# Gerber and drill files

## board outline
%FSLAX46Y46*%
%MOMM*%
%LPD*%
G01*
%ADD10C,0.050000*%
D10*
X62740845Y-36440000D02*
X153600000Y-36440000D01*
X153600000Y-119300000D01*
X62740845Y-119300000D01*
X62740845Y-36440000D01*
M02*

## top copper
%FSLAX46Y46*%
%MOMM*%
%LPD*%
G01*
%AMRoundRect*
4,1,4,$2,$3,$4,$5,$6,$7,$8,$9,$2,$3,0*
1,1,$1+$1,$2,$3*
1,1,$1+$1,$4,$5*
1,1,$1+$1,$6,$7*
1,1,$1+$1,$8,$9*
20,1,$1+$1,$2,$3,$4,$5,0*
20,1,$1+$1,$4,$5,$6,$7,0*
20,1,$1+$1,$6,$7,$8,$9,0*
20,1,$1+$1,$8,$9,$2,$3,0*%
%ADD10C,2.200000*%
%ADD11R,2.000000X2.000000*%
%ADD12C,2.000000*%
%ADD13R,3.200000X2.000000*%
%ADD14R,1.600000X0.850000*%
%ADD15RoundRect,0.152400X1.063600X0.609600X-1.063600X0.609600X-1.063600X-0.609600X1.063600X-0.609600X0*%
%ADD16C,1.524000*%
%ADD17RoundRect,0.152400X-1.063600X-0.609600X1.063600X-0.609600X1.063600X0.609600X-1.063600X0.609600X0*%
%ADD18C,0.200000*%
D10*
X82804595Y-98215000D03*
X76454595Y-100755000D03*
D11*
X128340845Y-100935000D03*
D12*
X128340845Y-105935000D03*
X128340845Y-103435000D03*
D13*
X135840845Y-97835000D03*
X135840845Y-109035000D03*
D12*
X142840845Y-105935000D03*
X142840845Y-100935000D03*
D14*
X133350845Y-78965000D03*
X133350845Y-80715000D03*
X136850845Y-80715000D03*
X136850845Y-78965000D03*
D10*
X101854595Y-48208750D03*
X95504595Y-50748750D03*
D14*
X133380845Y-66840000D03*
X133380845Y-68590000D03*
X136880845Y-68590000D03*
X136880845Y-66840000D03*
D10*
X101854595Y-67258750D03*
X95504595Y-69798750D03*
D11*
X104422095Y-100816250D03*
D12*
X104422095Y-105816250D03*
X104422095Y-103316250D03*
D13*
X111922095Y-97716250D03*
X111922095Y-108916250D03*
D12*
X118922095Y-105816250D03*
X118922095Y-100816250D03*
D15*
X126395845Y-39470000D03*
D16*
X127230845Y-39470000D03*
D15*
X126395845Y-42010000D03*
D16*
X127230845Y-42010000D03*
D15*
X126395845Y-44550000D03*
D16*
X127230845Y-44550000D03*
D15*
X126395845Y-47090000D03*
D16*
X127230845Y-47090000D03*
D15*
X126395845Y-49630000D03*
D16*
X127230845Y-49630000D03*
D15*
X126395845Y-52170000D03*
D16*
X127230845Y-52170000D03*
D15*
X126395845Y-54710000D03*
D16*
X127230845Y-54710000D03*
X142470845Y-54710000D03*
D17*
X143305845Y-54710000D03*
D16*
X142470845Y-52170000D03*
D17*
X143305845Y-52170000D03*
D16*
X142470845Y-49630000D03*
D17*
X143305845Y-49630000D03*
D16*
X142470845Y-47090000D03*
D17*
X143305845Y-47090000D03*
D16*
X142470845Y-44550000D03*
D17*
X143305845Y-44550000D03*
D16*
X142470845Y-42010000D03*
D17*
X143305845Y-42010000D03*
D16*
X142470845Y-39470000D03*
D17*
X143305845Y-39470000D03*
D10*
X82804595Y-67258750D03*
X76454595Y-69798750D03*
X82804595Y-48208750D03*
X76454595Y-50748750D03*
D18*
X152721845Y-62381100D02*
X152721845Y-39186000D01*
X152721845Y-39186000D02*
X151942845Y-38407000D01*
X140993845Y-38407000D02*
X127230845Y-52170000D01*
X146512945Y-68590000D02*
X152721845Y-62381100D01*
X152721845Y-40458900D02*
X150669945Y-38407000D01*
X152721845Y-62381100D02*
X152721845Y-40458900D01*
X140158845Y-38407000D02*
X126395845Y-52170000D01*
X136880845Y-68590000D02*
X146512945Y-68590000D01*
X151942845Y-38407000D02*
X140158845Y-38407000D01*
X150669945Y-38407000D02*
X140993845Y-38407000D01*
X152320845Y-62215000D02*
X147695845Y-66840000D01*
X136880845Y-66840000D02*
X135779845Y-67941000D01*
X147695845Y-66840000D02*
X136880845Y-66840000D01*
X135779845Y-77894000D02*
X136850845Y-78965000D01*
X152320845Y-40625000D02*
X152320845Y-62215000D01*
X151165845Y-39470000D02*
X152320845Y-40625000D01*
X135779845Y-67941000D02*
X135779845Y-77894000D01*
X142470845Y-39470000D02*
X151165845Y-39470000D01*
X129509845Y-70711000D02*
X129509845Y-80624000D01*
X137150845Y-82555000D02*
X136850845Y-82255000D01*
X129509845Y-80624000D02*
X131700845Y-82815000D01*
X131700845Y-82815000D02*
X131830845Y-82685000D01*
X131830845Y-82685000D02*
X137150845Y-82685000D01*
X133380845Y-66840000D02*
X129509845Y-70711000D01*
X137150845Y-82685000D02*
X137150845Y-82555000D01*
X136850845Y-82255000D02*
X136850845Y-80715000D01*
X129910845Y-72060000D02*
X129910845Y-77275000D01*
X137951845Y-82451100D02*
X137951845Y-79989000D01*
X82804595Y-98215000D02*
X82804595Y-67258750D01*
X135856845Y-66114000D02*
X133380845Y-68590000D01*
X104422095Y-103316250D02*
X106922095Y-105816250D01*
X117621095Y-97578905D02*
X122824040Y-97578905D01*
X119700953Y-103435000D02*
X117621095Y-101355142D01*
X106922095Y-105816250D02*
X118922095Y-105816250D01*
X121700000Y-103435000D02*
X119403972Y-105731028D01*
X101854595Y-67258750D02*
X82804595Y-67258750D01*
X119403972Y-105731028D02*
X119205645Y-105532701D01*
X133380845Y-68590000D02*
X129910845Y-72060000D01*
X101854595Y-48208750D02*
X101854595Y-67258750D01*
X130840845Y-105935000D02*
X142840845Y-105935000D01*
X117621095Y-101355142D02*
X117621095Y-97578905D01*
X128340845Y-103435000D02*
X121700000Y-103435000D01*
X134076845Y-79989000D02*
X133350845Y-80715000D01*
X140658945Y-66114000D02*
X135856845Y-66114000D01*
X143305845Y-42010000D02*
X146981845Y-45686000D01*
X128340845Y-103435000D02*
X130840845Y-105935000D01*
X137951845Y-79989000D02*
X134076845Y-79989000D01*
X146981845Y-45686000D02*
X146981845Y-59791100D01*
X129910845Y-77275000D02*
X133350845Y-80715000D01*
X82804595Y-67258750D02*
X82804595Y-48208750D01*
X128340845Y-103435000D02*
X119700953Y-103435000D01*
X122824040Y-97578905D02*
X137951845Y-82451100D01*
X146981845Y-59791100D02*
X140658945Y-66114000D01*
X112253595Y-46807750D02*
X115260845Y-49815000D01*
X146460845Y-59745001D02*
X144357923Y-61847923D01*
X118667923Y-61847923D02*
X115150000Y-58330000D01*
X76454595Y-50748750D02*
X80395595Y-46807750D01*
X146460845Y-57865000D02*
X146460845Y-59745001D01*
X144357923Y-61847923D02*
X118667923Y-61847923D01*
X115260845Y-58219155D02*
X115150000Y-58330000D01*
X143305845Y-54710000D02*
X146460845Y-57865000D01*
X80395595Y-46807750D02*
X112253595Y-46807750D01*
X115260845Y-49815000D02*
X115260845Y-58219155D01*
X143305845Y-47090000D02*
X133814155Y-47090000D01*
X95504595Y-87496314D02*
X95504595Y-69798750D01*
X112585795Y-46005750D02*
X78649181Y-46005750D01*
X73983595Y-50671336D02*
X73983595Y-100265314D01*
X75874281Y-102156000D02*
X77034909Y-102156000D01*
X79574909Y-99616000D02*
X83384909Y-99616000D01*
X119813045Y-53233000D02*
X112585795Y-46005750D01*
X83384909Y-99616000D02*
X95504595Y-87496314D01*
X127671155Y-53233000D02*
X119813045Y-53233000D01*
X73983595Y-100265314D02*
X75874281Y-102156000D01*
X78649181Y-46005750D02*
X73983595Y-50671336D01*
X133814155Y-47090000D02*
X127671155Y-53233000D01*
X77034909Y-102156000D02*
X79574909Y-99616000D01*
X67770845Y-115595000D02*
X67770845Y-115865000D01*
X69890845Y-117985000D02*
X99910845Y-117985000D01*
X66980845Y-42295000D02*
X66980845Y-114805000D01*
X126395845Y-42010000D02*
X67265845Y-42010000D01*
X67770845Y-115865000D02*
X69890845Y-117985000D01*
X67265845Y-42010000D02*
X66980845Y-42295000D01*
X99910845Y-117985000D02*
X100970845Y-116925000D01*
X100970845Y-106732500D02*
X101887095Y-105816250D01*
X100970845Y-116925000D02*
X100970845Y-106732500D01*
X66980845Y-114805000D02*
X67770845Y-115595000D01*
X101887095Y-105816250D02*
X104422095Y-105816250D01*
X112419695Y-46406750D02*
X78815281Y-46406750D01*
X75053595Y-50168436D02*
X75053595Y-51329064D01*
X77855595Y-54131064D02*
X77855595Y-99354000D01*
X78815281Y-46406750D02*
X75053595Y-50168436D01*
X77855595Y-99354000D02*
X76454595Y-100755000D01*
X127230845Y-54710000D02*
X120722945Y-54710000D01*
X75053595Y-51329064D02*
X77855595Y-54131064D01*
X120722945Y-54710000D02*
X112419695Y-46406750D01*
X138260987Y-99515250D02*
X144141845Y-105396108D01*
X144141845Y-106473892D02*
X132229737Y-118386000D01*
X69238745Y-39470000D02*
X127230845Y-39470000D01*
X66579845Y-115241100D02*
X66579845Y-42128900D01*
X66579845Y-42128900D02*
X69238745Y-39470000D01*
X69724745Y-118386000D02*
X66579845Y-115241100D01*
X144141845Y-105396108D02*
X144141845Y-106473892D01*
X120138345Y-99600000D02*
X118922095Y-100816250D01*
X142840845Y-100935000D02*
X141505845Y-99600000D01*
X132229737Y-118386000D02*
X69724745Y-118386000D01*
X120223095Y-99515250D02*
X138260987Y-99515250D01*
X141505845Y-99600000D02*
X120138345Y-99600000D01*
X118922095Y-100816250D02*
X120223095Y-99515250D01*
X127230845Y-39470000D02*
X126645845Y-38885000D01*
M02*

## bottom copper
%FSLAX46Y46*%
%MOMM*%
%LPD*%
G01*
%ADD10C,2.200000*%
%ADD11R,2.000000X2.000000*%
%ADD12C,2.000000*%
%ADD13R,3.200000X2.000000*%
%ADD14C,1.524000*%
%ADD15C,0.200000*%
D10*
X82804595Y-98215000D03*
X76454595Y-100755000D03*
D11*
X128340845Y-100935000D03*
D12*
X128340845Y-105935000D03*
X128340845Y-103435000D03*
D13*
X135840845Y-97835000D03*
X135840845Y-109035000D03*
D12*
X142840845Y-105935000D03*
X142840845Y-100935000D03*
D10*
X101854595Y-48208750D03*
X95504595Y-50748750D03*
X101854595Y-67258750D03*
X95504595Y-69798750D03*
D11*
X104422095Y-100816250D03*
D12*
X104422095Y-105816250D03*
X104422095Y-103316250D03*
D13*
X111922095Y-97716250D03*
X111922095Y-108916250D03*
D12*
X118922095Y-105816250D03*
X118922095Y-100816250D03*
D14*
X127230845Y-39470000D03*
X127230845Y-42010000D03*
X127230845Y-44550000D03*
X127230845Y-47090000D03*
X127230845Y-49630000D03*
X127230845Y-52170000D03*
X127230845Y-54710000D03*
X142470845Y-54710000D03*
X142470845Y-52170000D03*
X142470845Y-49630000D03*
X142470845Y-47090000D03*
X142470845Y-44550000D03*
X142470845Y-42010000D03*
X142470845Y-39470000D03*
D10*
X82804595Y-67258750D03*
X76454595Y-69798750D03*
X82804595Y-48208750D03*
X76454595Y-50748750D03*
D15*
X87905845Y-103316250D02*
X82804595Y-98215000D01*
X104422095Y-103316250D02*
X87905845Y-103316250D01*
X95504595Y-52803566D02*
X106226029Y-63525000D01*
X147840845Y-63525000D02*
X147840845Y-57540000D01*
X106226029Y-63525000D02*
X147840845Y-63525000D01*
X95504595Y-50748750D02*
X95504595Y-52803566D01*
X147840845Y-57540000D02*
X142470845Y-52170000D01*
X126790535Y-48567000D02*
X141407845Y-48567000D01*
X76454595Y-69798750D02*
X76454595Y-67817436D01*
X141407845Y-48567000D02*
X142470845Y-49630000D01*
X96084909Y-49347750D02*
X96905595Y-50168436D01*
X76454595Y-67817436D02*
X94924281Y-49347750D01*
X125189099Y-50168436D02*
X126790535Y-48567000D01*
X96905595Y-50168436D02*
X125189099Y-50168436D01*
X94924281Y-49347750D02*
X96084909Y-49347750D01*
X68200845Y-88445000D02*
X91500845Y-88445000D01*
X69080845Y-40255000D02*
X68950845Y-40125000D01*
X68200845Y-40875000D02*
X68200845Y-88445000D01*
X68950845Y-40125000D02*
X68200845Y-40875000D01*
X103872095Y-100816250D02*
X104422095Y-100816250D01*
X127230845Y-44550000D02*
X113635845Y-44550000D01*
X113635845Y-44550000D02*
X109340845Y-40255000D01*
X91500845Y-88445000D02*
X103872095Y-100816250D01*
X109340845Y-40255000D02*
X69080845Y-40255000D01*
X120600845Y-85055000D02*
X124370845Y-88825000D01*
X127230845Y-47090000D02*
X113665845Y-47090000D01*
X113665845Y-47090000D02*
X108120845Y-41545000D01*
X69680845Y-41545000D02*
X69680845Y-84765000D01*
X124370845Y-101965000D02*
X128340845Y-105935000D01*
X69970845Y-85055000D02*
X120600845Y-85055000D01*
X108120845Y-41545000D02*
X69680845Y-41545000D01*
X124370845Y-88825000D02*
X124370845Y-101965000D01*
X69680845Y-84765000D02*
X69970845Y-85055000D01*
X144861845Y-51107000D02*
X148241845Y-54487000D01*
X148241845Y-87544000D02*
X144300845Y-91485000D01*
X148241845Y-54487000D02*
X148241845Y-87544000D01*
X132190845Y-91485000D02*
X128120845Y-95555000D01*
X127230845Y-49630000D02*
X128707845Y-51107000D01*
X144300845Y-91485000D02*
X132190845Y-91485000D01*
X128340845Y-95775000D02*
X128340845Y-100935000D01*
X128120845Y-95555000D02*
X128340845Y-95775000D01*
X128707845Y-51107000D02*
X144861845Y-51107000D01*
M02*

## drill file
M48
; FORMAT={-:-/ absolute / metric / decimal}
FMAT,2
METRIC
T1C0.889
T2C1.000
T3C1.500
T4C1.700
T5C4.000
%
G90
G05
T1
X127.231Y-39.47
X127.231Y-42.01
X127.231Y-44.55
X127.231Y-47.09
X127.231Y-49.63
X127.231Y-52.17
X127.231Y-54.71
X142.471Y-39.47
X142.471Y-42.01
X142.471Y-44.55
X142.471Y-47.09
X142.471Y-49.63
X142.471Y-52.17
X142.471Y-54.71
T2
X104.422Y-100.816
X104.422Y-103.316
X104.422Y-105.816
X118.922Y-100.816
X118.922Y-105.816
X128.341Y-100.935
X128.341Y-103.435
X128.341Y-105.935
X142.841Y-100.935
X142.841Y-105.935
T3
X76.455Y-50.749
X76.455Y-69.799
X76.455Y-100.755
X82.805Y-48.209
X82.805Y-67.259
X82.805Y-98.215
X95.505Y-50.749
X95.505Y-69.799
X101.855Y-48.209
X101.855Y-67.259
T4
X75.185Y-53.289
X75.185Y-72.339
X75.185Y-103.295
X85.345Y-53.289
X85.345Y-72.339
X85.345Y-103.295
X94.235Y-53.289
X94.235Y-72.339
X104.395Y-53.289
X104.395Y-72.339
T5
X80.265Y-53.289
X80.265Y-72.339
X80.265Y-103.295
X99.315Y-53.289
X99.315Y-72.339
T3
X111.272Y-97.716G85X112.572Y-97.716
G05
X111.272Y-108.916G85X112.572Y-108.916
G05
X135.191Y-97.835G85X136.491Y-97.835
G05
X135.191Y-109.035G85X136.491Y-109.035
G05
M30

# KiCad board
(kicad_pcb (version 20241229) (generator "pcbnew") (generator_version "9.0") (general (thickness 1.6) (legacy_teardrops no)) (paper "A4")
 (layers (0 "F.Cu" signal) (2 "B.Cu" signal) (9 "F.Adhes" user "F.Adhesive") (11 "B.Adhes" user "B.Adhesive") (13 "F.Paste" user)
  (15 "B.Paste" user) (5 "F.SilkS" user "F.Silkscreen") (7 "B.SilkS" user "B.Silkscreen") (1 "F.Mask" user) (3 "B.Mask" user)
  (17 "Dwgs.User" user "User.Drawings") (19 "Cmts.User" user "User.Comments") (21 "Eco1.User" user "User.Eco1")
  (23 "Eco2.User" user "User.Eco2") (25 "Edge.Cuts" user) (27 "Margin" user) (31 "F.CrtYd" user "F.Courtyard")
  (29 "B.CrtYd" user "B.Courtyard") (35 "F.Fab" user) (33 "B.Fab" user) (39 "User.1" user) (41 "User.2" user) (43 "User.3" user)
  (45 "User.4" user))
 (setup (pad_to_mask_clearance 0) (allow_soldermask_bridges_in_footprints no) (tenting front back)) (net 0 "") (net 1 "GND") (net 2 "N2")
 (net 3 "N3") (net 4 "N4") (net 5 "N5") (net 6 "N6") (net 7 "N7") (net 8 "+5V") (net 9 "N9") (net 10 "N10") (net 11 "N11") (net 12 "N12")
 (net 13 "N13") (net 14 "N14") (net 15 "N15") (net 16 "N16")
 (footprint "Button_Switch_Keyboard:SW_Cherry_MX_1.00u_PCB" (layer "F.Cu") (at 82.804595 98.215)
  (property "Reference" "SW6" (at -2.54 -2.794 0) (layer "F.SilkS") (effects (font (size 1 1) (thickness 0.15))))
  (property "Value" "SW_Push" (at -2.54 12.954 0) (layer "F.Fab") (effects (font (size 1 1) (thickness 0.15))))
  (pad "" np_thru_hole circle (at -7.62 5.08) (size 1.7 1.7) (drill 1.7) (layers "*.Cu" "*.Mask"))
  (pad "" np_thru_hole circle (at -2.54 5.08) (size 4 4) (drill 4) (layers "*.Cu" "*.Mask"))
  (pad "" np_thru_hole circle (at 2.54 5.08) (size 1.7 1.7) (drill 1.7) (layers "*.Cu" "*.Mask"))
  (pad "1" thru_hole circle (at 0 0) (size 2.2 2.2) (drill 1.5) (layers "*.Cu" "*.Mask") (remove_unused_layers no) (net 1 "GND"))
  (pad "2" thru_hole circle (at -6.35 2.54) (size 2.2 2.2) (drill 1.5) (layers "*.Cu" "*.Mask") (remove_unused_layers no) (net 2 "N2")))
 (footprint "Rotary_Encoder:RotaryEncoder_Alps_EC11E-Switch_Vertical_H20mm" (layer "F.Cu") (at 128.340845 100.935)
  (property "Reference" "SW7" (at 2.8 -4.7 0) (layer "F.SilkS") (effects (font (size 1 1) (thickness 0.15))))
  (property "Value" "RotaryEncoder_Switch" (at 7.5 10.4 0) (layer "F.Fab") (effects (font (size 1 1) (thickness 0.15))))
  (pad "A" thru_hole rect (at 0 0) (size 2 2) (drill 1) (layers "*.Cu" "*.Mask") (remove_unused_layers no) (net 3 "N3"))
  (pad "B" thru_hole circle (at 0 5) (size 2 2) (drill 1) (layers "*.Cu" "*.Mask") (remove_unused_layers no) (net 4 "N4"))
  (pad "C" thru_hole circle (at 0 2.5) (size 2 2) (drill 1) (layers "*.Cu" "*.Mask") (remove_unused_layers no) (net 1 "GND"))
  (pad "MP" thru_hole rect (at 7.5 -3.1) (size 3.2 2) (drill oval 2.8 1.5) (layers "*.Cu" "*.Mask") (remove_unused_layers no))
  (pad "MP" thru_hole rect (at 7.5 8.1) (size 3.2 2) (drill oval 2.8 1.5) (layers "*.Cu" "*.Mask") (remove_unused_layers no))
  (pad "S1" thru_hole circle (at 14.5 5) (size 2 2) (drill 1) (layers "*.Cu" "*.Mask") (remove_unused_layers no) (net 1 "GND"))
  (pad "S2" thru_hole circle (at 14.5 0) (size 2 2) (drill 1) (layers "*.Cu" "*.Mask") (remove_unused_layers no) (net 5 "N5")))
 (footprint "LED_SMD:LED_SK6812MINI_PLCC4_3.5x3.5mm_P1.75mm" (layer "F.Cu") (at 135.100845 79.84)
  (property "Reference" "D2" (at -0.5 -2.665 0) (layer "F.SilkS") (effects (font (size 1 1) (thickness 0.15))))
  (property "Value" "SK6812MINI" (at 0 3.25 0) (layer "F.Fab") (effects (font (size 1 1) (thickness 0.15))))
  (pad "1" smd rect (at -1.75 -0.875) (size 1.6 0.85) (layers "F.Cu" "F.Mask" "F.Paste") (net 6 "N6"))
  (pad "2" smd rect (at -1.75 0.875) (size 1.6 0.85) (layers "F.Cu" "F.Mask" "F.Paste") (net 1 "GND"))
  (pad "3" smd rect (at 1.75 0.875) (size 1.6 0.85) (layers "F.Cu" "F.Mask" "F.Paste") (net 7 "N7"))
  (pad "4" smd rect (at 1.75 -0.875) (size 1.6 0.85) (layers "F.Cu" "F.Mask" "F.Paste") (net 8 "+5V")))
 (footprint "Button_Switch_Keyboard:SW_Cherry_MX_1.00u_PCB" (layer "F.Cu") (at 101.854595 48.20875)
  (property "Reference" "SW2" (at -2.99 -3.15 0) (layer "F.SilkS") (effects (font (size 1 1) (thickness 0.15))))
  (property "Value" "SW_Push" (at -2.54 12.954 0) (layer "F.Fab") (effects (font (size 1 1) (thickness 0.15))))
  (pad "" np_thru_hole circle (at -7.62 5.08) (size 1.7 1.7) (drill 1.7) (layers "*.Cu" "*.Mask"))
  (pad "" np_thru_hole circle (at -2.54 5.08) (size 4 4) (drill 4) (layers "*.Cu" "*.Mask"))
  (pad "" np_thru_hole circle (at 2.54 5.08) (size 1.7 1.7) (drill 1.7) (layers "*.Cu" "*.Mask"))
  (pad "1" thru_hole circle (at 0 0) (size 2.2 2.2) (drill 1.5) (layers "*.Cu" "*.Mask") (remove_unused_layers no) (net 1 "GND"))
  (pad "2" thru_hole circle (at -6.35 2.54) (size 2.2 2.2) (drill 1.5) (layers "*.Cu" "*.Mask") (remove_unused_layers no) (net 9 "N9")))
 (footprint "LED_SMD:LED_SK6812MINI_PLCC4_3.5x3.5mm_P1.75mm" (layer "F.Cu") (at 135.130845 67.715)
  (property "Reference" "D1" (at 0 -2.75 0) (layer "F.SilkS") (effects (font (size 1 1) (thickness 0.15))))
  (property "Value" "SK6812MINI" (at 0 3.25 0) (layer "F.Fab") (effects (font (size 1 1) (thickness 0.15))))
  (pad "1" smd rect (at -1.75 -0.875) (size 1.6 0.85) (layers "F.Cu" "F.Mask" "F.Paste") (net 7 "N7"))
  (pad "2" smd rect (at -1.75 0.875) (size 1.6 0.85) (layers "F.Cu" "F.Mask" "F.Paste") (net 1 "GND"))
  (pad "3" smd rect (at 1.75 0.875) (size 1.6 0.85) (layers "F.Cu" "F.Mask" "F.Paste") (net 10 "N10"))
  (pad "4" smd rect (at 1.75 -0.875) (size 1.6 0.85) (layers "F.Cu" "F.Mask" "F.Paste") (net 8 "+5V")))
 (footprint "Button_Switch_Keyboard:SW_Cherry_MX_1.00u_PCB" (layer "F.Cu") (at 101.854595 67.25875)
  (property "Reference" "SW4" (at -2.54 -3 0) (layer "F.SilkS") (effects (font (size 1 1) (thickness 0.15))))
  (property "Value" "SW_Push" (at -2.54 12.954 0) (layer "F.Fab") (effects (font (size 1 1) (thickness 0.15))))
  (pad "" np_thru_hole circle (at -7.62 5.08) (size 1.7 1.7) (drill 1.7) (layers "*.Cu" "*.Mask"))
  (pad "" np_thru_hole circle (at -2.54 5.08) (size 4 4) (drill 4) (layers "*.Cu" "*.Mask"))
  (pad "" np_thru_hole circle (at 2.54 5.08) (size 1.7 1.7) (drill 1.7) (layers "*.Cu" "*.Mask"))
  (pad "1" thru_hole circle (at 0 0) (size 2.2 2.2) (drill 1.5) (layers "*.Cu" "*.Mask") (remove_unused_layers no) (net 1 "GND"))
  (pad "2" thru_hole circle (at -6.35 2.54) (size 2.2 2.2) (drill 1.5) (layers "*.Cu" "*.Mask") (remove_unused_layers no) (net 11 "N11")))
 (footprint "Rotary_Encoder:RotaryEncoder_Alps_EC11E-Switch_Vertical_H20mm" (layer "F.Cu") (at 104.422095 100.81625)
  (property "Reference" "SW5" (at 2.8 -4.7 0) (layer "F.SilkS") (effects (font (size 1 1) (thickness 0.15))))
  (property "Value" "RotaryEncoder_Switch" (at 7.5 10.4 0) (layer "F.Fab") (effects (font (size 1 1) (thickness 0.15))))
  (pad "A" thru_hole rect (at 0 0) (size 2 2) (drill 1) (layers "*.Cu" "*.Mask") (remove_unused_layers no) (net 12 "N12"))
  (pad "B" thru_hole circle (at 0 5) (size 2 2) (drill 1) (layers "*.Cu" "*.Mask") (remove_unused_layers no) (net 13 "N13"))
  (pad "C" thru_hole circle (at 0 2.5) (size 2 2) (drill 1) (layers "*.Cu" "*.Mask") (remove_unused_layers no) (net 1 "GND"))
  (pad "MP" thru_hole rect (at 7.5 -3.1) (size 3.2 2) (drill oval 2.8 1.5) (layers "*.Cu" "*.Mask") (remove_unused_layers no))
  (pad "MP" thru_hole rect (at 7.5 8.1) (size 3.2 2) (drill oval 2.8 1.5) (layers "*.Cu" "*.Mask") (remove_unused_layers no))
  (pad "S1" thru_hole circle (at 14.5 5) (size 2 2) (drill 1) (layers "*.Cu" "*.Mask") (remove_unused_layers no) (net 1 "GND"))
  (pad "S2" thru_hole circle (at 14.5 0) (size 2 2) (drill 1) (layers "*.Cu" "*.Mask") (remove_unused_layers no) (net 5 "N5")))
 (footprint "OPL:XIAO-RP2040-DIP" (layer "F.Cu") (at 134.850845 47.09)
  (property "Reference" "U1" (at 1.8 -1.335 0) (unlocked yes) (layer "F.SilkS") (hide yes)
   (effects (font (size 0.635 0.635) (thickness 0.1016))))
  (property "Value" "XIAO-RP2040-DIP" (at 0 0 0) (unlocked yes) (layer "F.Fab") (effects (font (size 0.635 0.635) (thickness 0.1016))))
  (pad "1" smd roundrect (at -8.455 -7.62 180) (size 2.432 1.524) (layers "F.Cu" "F.Mask") (roundrect_rratio 0.1) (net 5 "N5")
   (thermal_bridge_angle 45))
  (pad "1" thru_hole circle (at -7.62 -7.62 180) (size 1.524 1.524) (drill 0.889) (layers "*.Cu" "*.Mask") (remove_unused_layers no)
   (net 5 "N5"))
  (pad "2" smd roundrect (at -8.455 -5.08 180) (size 2.432 1.524) (layers "F.Cu" "F.Mask") (roundrect_rratio 0.1) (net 13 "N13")
   (thermal_bridge_angle 45))
  (pad "2" thru_hole circle (at -7.62 -5.08 180) (size 1.524 1.524) (drill 0.889) (layers "*.Cu" "*.Mask") (remove_unused_layers no)
   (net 13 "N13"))
  (pad "3" smd roundrect (at -8.455 -2.54 180) (size 2.432 1.524) (layers "F.Cu" "F.Mask") (roundrect_rratio 0.1) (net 12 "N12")
   (thermal_bridge_angle 45))
  (pad "3" thru_hole circle (at -7.62 -2.54 180) (size 1.524 1.524) (drill 0.889) (layers "*.Cu" "*.Mask") (remove_unused_layers no)
   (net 12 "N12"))
  (pad "4" smd roundrect (at -8.455 0 180) (size 2.432 1.524) (layers "F.Cu" "F.Mask") (roundrect_rratio 0.1) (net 4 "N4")
   (thermal_bridge_angle 45))
  (pad "4" thru_hole circle (at -7.62 0 180) (size 1.524 1.524) (drill 0.889) (layers "*.Cu" "*.Mask") (remove_unused_layers no)
   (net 4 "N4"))
  (pad "5" smd roundrect (at -8.455 2.54 180) (size 2.432 1.524) (layers "F.Cu" "F.Mask") (roundrect_rratio 0.1) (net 3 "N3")
   (thermal_bridge_angle 45))
  (pad "5" thru_hole circle (at -7.62 2.54 180) (size 1.524 1.524) (drill 0.889) (layers "*.Cu" "*.Mask") (remove_unused_layers no)
   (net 3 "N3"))
  (pad "6" smd roundrect (at -8.455 5.08 180) (size 2.432 1.524) (layers "F.Cu" "F.Mask") (roundrect_rratio 0.1) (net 10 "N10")
   (thermal_bridge_angle 45))
  (pad "6" thru_hole circle (at -7.62 5.08 180) (size 1.524 1.524) (drill 0.889) (layers "*.Cu" "*.Mask") (remove_unused_layers no)
   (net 10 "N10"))
  (pad "7" smd roundrect (at -8.455 7.62 180) (size 2.432 1.524) (layers "F.Cu" "F.Mask") (roundrect_rratio 0.1) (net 2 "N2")
   (thermal_bridge_angle 45))
  (pad "7" thru_hole circle (at -7.62 7.62 180) (size 1.524 1.524) (drill 0.889) (layers "*.Cu" "*.Mask") (remove_unused_layers no)
   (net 2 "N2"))
  (pad "8" thru_hole circle (at 7.62 7.62) (size 1.524 1.524) (drill 0.889) (layers "*.Cu" "*.Mask") (remove_unused_layers no)
   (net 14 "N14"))
  (pad "8" smd roundrect (at 8.455 7.62) (size 2.432 1.524) (layers "F.Cu" "F.Mask") (roundrect_rratio 0.1) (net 14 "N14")
   (thermal_bridge_angle 45))
  (pad "9" thru_hole circle (at 7.62 5.08) (size 1.524 1.524) (drill 0.889) (layers "*.Cu" "*.Mask") (remove_unused_layers no) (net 9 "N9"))
  (pad "9" smd roundrect (at 8.455 5.08) (size 2.432 1.524) (layers "F.Cu" "F.Mask") (roundrect_rratio 0.1) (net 9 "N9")
   (thermal_bridge_angle 45))
  (pad "10" thru_hole circle (at 7.62 2.54) (size 1.524 1.524) (drill 0.889) (layers "*.Cu" "*.Mask") (remove_unused_layers no)
   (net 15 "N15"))
  (pad "10" smd roundrect (at 8.455 2.54) (size 2.432 1.524) (layers "F.Cu" "F.Mask") (roundrect_rratio 0.1) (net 15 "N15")
   (thermal_bridge_angle 45))
  (pad "11" thru_hole circle (at 7.62 0) (size 1.524 1.524) (drill 0.889) (layers "*.Cu" "*.Mask") (remove_unused_layers no) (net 11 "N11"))
  (pad "11" smd roundrect (at 8.455 0) (size 2.432 1.524) (layers "F.Cu" "F.Mask") (roundrect_rratio 0.1) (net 11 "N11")
   (thermal_bridge_angle 45))
  (pad "12" thru_hole circle (at 7.62 -2.54) (size 1.524 1.524) (drill 0.889) (layers "*.Cu" "*.Mask") (remove_unused_layers no)
   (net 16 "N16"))
  (pad "12" smd roundrect (at 8.455 -2.54) (size 2.432 1.524) (layers "F.Cu" "F.Mask") (roundrect_rratio 0.1) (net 16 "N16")
   (thermal_bridge_angle 45))
  (pad "13" thru_hole circle (at 7.62 -5.08) (size 1.524 1.524) (drill 0.889) (layers "*.Cu" "*.Mask") (remove_unused_layers no)
   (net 1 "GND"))
  (pad "13" smd roundrect (at 8.455 -5.08) (size 2.432 1.524) (layers "F.Cu" "F.Mask") (roundrect_rratio 0.1) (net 1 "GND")
   (thermal_bridge_angle 45))
  (pad "14" thru_hole circle (at 7.62 -7.62) (size 1.524 1.524) (drill 0.889) (layers "*.Cu" "*.Mask") (remove_unused_layers no)
   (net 8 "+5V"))
  (pad "14" smd roundrect (at 8.455 -7.62) (size 2.432 1.524) (layers "F.Cu" "F.Mask") (roundrect_rratio 0.1) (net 8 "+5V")
   (thermal_bridge_angle 45)))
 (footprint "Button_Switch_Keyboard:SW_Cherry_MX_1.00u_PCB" (layer "F.Cu") (at 82.804595 67.25875)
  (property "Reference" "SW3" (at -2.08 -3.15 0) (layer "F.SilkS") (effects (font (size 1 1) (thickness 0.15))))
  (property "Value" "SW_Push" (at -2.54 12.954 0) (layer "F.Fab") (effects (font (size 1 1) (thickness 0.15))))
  (pad "" np_thru_hole circle (at -7.62 5.08) (size 1.7 1.7) (drill 1.7) (layers "*.Cu" "*.Mask"))
  (pad "" np_thru_hole circle (at -2.54 5.08) (size 4 4) (drill 4) (layers "*.Cu" "*.Mask"))
  (pad "" np_thru_hole circle (at 2.54 5.08) (size 1.7 1.7) (drill 1.7) (layers "*.Cu" "*.Mask"))
  (pad "1" thru_hole circle (at 0 0) (size 2.2 2.2) (drill 1.5) (layers "*.Cu" "*.Mask") (remove_unused_layers no) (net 1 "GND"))
  (pad "2" thru_hole circle (at -6.35 2.54) (size 2.2 2.2) (drill 1.5) (layers "*.Cu" "*.Mask") (remove_unused_layers no) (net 15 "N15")))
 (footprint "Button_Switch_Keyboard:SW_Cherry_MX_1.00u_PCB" (layer "F.Cu") (at 82.804595 48.20875)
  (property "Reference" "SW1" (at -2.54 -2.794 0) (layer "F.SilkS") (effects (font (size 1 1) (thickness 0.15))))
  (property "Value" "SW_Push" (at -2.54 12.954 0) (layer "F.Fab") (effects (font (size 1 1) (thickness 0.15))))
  (pad "" np_thru_hole circle (at -7.62 5.08) (size 1.7 1.7) (drill 1.7) (layers "*.Cu" "*.Mask"))
  (pad "" np_thru_hole circle (at -2.54 5.08) (size 4 4) (drill 4) (layers "*.Cu" "*.Mask"))
  (pad "" np_thru_hole circle (at 2.54 5.08) (size 1.7 1.7) (drill 1.7) (layers "*.Cu" "*.Mask"))
  (pad "1" thru_hole circle (at 0 0) (size 2.2 2.2) (drill 1.5) (layers "*.Cu" "*.Mask") (remove_unused_layers no) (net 1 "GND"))
  (pad "2" thru_hole circle (at -6.35 2.54) (size 2.2 2.2) (drill 1.5) (layers "*.Cu" "*.Mask") (remove_unused_layers no) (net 14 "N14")))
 (gr_rect (start 62.740845 36.44) (end 153.6 119.3) (stroke (width 0.05) (type default)) (fill no) (layer "Edge.Cuts"))
 (segment (start 152.721845 62.3811) (end 152.721845 39.186) (width 0.2) (layer "F.Cu") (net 10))
 (segment (start 152.721845 39.186) (end 151.942845 38.407) (width 0.2) (layer "F.Cu") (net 10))
 (segment (start 140.993845 38.407) (end 127.230845 52.17) (width 0.2) (layer "F.Cu") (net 10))
 (segment (start 146.512945 68.59) (end 152.721845 62.3811) (width 0.2) (layer "F.Cu") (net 10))
 (segment (start 152.721845 40.4589) (end 150.669945 38.407) (width 0.2) (layer "F.Cu") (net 10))
 (segment (start 152.721845 62.3811) (end 152.721845 40.4589) (width 0.2) (layer "F.Cu") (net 10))
 (segment (start 140.158845 38.407) (end 126.395845 52.17) (width 0.2) (layer "F.Cu") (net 10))
 (segment (start 136.880845 68.59) (end 146.512945 68.59) (width 0.2) (layer "F.Cu") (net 10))
 (segment (start 151.942845 38.407) (end 140.158845 38.407) (width 0.2) (layer "F.Cu") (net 10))
 (segment (start 150.669945 38.407) (end 140.993845 38.407) (width 0.2) (layer "F.Cu") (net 10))
 (segment (start 152.320845 62.215) (end 147.695845 66.84) (width 0.2) (layer "F.Cu") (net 8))
 (segment (start 136.880845 66.84) (end 135.779845 67.941) (width 0.2) (layer "F.Cu") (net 8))
 (segment (start 147.695845 66.84) (end 136.880845 66.84) (width 0.2) (layer "F.Cu") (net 8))
 (segment (start 135.779845 77.894) (end 136.850845 78.965) (width 0.2) (layer "F.Cu") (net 8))
 (segment (start 152.320845 40.625) (end 152.320845 62.215) (width 0.2) (layer "F.Cu") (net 8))
 (segment (start 151.165845 39.47) (end 152.320845 40.625) (width 0.2) (layer "F.Cu") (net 8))
 (segment (start 135.779845 67.941) (end 135.779845 77.894) (width 0.2) (layer "F.Cu") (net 8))
 (segment (start 142.470845 39.47) (end 151.165845 39.47) (width 0.2) (layer "F.Cu") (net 8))
 (segment (start 129.509845 70.711) (end 129.509845 80.624) (width 0.2) (layer "F.Cu") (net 7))
 (segment (start 137.150845 82.555) (end 136.850845 82.255) (width 0.2) (layer "F.Cu") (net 7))
 (segment (start 129.509845 80.624) (end 131.700845 82.815) (width 0.2) (layer "F.Cu") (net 7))
 (segment (start 131.700845 82.815) (end 131.830845 82.685) (width 0.2) (layer "F.Cu") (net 7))
 (segment (start 131.830845 82.685) (end 137.150845 82.685) (width 0.2) (layer "F.Cu") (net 7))
 (segment (start 133.380845 66.84) (end 129.509845 70.711) (width 0.2) (layer "F.Cu") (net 7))
 (segment (start 137.150845 82.685) (end 137.150845 82.555) (width 0.2) (layer "F.Cu") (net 7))
 (segment (start 136.850845 82.255) (end 136.850845 80.715) (width 0.2) (layer "F.Cu") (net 7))
 (segment (start 129.910845 72.06) (end 129.910845 77.275) (width 0.2) (layer "F.Cu") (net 1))
 (segment (start 137.951845 82.4511) (end 137.951845 79.989) (width 0.2) (layer "F.Cu") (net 1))
 (segment (start 82.804595 98.215) (end 82.804595 67.25875) (width 0.2) (layer "F.Cu") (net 1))
 (segment (start 135.856845 66.114) (end 133.380845 68.59) (width 0.2) (layer "F.Cu") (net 1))
 (segment (start 104.422095 103.31625) (end 106.922095 105.81625) (width 0.2) (layer "F.Cu") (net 1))
 (segment (start 117.621095 97.578905) (end 122.82404 97.578905) (width 0.2) (layer "F.Cu") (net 1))
 (segment (start 119.700953 103.435) (end 117.621095 101.355142) (width 0.2) (layer "F.Cu") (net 1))
 (segment (start 106.922095 105.81625) (end 118.922095 105.81625) (width 0.2) (layer "F.Cu") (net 1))
 (segment (start 121.7 103.435) (end 119.403972 105.731028) (width 0.2) (layer "F.Cu") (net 1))
 (segment (start 101.854595 67.25875) (end 82.804595 67.25875) (width 0.2) (layer "F.Cu") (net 1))
 (segment (start 119.403972 105.731028) (end 119.205645 105.532701) (width 0.2) (layer "F.Cu") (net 1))
 (segment (start 133.380845 68.59) (end 129.910845 72.06) (width 0.2) (layer "F.Cu") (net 1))
 (segment (start 101.854595 48.20875) (end 101.854595 67.25875) (width 0.2) (layer "F.Cu") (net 1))
 (segment (start 130.840845 105.935) (end 142.840845 105.935) (width 0.2) (layer "F.Cu") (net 1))
 (segment (start 117.621095 101.355142) (end 117.621095 97.578905) (width 0.2) (layer "F.Cu") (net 1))
 (segment (start 128.340845 103.435) (end 121.7 103.435) (width 0.2) (layer "F.Cu") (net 1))
 (segment (start 134.076845 79.989) (end 133.350845 80.715) (width 0.2) (layer "F.Cu") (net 1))
 (segment (start 140.658945 66.114) (end 135.856845 66.114) (width 0.2) (layer "F.Cu") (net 1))
 (segment (start 143.305845 42.01) (end 146.981845 45.686) (width 0.2) (layer "F.Cu") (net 1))
 (segment (start 128.340845 103.435) (end 130.840845 105.935) (width 0.2) (layer "F.Cu") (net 1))
 (segment (start 137.951845 79.989) (end 134.076845 79.989) (width 0.2) (layer "F.Cu") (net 1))
 (segment (start 146.981845 45.686) (end 146.981845 59.7911) (width 0.2) (layer "F.Cu") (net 1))
 (segment (start 129.910845 77.275) (end 133.350845 80.715) (width 0.2) (layer "F.Cu") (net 1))
 (segment (start 82.804595 67.25875) (end 82.804595 48.20875) (width 0.2) (layer "F.Cu") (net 1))
 (segment (start 128.340845 103.435) (end 119.700953 103.435) (width 0.2) (layer "F.Cu") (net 1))
 (segment (start 122.82404 97.578905) (end 137.951845 82.4511) (width 0.2) (layer "F.Cu") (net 1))
 (segment (start 146.981845 59.7911) (end 140.658945 66.114) (width 0.2) (layer "F.Cu") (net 1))
 (segment (start 87.905845 103.31625) (end 82.804595 98.215) (width 0.2) (layer "B.Cu") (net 1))
 (segment (start 104.422095 103.31625) (end 87.905845 103.31625) (width 0.2) (layer "B.Cu") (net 1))
 (segment (start 112.253595 46.80775) (end 115.260845 49.815) (width 0.2) (layer "F.Cu") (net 14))
 (segment (start 146.460845 59.745001) (end 144.357923 61.847923) (width 0.2) (layer "F.Cu") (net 14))
 (segment (start 118.667923 61.847923) (end 115.15 58.33) (width 0.2) (layer "F.Cu") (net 14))
 (segment (start 76.454595 50.74875) (end 80.395595 46.80775) (width 0.2) (layer "F.Cu") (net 14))
 (segment (start 146.460845 57.865) (end 146.460845 59.745001) (width 0.2) (layer "F.Cu") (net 14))
 (segment (start 144.357923 61.847923) (end 118.667923 61.847923) (width 0.2) (layer "F.Cu") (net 14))
 (segment (start 115.260845 58.219155) (end 115.15 58.33) (width 0.2) (layer "F.Cu") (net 14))
 (segment (start 143.305845 54.71) (end 146.460845 57.865) (width 0.2) (layer "F.Cu") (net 14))
 (segment (start 80.395595 46.80775) (end 112.253595 46.80775) (width 0.2) (layer "F.Cu") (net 14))
 (segment (start 115.260845 49.815) (end 115.260845 58.219155) (width 0.2) (layer "F.Cu") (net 14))
 (segment (start 95.504595 52.803566) (end 106.226029 63.525) (width 0.2) (layer "B.Cu") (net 9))
 (segment (start 147.840845 63.525) (end 147.840845 57.54) (width 0.2) (layer "B.Cu") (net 9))
 (segment (start 106.226029 63.525) (end 147.840845 63.525) (width 0.2) (layer "B.Cu") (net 9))
 (segment (start 95.504595 50.74875) (end 95.504595 52.803566) (width 0.2) (layer "B.Cu") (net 9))
 (segment (start 147.840845 57.54) (end 142.470845 52.17) (width 0.2) (layer "B.Cu") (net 9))
 (segment (start 126.790535 48.567) (end 141.407845 48.567) (width 0.2) (layer "B.Cu") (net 15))
 (segment (start 76.454595 69.79875) (end 76.454595 67.817436) (width 0.2) (layer "B.Cu") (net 15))
 (segment (start 141.407845 48.567) (end 142.470845 49.63) (width 0.2) (layer "B.Cu") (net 15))
 (segment (start 96.084909 49.34775) (end 96.905595 50.168436) (width 0.2) (layer "B.Cu") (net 15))
 (segment (start 76.454595 67.817436) (end 94.924281 49.34775) (width 0.2) (layer "B.Cu") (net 15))
 (segment (start 125.189099 50.168436) (end 126.790535 48.567) (width 0.2) (layer "B.Cu") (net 15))
 (segment (start 96.905595 50.168436) (end 125.189099 50.168436) (width 0.2) (layer "B.Cu") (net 15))
 (segment (start 94.924281 49.34775) (end 96.084909 49.34775) (width 0.2) (layer "B.Cu") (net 15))
 (segment (start 143.305845 47.09) (end 133.814155 47.09) (width 0.2) (layer "F.Cu") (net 11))
 (segment (start 95.504595 87.496314) (end 95.504595 69.79875) (width 0.2) (layer "F.Cu") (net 11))
 (segment (start 112.585795 46.00575) (end 78.649181 46.00575) (width 0.2) (layer "F.Cu") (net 11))
 (segment (start 73.983595 50.671336) (end 73.983595 100.265314) (width 0.2) (layer "F.Cu") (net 11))
 (segment (start 75.874281 102.156) (end 77.034909 102.156) (width 0.2) (layer "F.Cu") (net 11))
 (segment (start 79.574909 99.616) (end 83.384909 99.616) (width 0.2) (layer "F.Cu") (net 11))
 (segment (start 119.813045 53.233) (end 112.585795 46.00575) (width 0.2) (layer "F.Cu") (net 11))
 (segment (start 83.384909 99.616) (end 95.504595 87.496314) (width 0.2) (layer "F.Cu") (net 11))
 (segment (start 127.671155 53.233) (end 119.813045 53.233) (width 0.2) (layer "F.Cu") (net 11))
 (segment (start 73.983595 100.265314) (end 75.874281 102.156) (width 0.2) (layer "F.Cu") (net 11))
 (segment (start 78.649181 46.00575) (end 73.983595 50.671336) (width 0.2) (layer "F.Cu") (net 11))
 (segment (start 133.814155 47.09) (end 127.671155 53.233) (width 0.2) (layer "F.Cu") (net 11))
 (segment (start 77.034909 102.156) (end 79.574909 99.616) (width 0.2) (layer "F.Cu") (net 11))
 (segment (start 67.770845 115.595) (end 67.770845 115.865) (width 0.2) (layer "F.Cu") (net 13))
 (segment (start 69.890845 117.985) (end 99.910845 117.985) (width 0.2) (layer "F.Cu") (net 13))
 (segment (start 66.980845 42.295) (end 66.980845 114.805) (width 0.2) (layer "F.Cu") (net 13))
 (segment (start 126.395845 42.01) (end 67.265845 42.01) (width 0.2) (layer "F.Cu") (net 13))
 (segment (start 67.770845 115.865) (end 69.890845 117.985) (width 0.2) (layer "F.Cu") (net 13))
 (segment (start 67.265845 42.01) (end 66.980845 42.295) (width 0.2) (layer "F.Cu") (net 13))
 (segment (start 99.910845 117.985) (end 100.970845 116.925) (width 0.2) (layer "F.Cu") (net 13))
 (segment (start 100.970845 106.7325) (end 101.887095 105.81625) (width 0.2) (layer "F.Cu") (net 13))
 (segment (start 100.970845 116.925) (end 100.970845 106.7325) (width 0.2) (layer "F.Cu") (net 13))
 (segment (start 66.980845 114.805) (end 67.770845 115.595) (width 0.2) (layer "F.Cu") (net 13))
 (segment (start 101.887095 105.81625) (end 104.422095 105.81625) (width 0.2) (layer "F.Cu") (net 13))
 (segment (start 112.419695 46.40675) (end 78.815281 46.40675) (width 0.2) (layer "F.Cu") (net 2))
 (segment (start 75.053595 50.168436) (end 75.053595 51.329064) (width 0.2) (layer "F.Cu") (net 2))
 (segment (start 77.855595 54.131064) (end 77.855595 99.354) (width 0.2) (layer "F.Cu") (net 2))
 (segment (start 78.815281 46.40675) (end 75.053595 50.168436) (width 0.2) (layer "F.Cu") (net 2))
 (segment (start 77.855595 99.354) (end 76.454595 100.755) (width 0.2) (layer "F.Cu") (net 2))
 (segment (start 127.230845 54.71) (end 120.722945 54.71) (width 0.2) (layer "F.Cu") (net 2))
 (segment (start 75.053595 51.329064) (end 77.855595 54.131064) (width 0.2) (layer "F.Cu") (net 2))
 (segment (start 120.722945 54.71) (end 112.419695 46.40675) (width 0.2) (layer "F.Cu") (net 2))
 (segment (start 68.200845 88.445) (end 91.500845 88.445) (width 0.2) (layer "B.Cu") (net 12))
 (segment (start 69.080845 40.255) (end 68.950845 40.125) (width 0.2) (layer "B.Cu") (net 12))
 (segment (start 68.200845 40.875) (end 68.200845 88.445) (width 0.2) (layer "B.Cu") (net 12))
 (segment (start 68.950845 40.125) (end 68.200845 40.875) (width 0.2) (layer "B.Cu") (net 12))
 (segment (start 103.872095 100.81625) (end 104.422095 100.81625) (width 0.2) (layer "B.Cu") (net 12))
 (segment (start 127.230845 44.55) (end 113.635845 44.55) (width 0.2) (layer "B.Cu") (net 12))
 (segment (start 113.635845 44.55) (end 109.340845 40.255) (width 0.2) (layer "B.Cu") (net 12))
 (segment (start 91.500845 88.445) (end 103.872095 100.81625) (width 0.2) (layer "B.Cu") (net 12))
 (segment (start 109.340845 40.255) (end 69.080845 40.255) (width 0.2) (layer "B.Cu") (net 12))
 (segment (start 120.600845 85.055) (end 124.370845 88.825) (width 0.2) (layer "B.Cu") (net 4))
 (segment (start 127.230845 47.09) (end 113.665845 47.09) (width 0.2) (layer "B.Cu") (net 4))
 (segment (start 113.665845 47.09) (end 108.120845 41.545) (width 0.2) (layer "B.Cu") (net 4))
 (segment (start 69.680845 41.545) (end 69.680845 84.765) (width 0.2) (layer "B.Cu") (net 4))
 (segment (start 124.370845 101.965) (end 128.340845 105.935) (width 0.2) (layer "B.Cu") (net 4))
 (segment (start 69.970845 85.055) (end 120.600845 85.055) (width 0.2) (layer "B.Cu") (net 4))
 (segment (start 108.120845 41.545) (end 69.680845 41.545) (width 0.2) (layer "B.Cu") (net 4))
 (segment (start 124.370845 88.825) (end 124.370845 101.965) (width 0.2) (layer "B.Cu") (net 4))
 (segment (start 69.680845 84.765) (end 69.970845 85.055) (width 0.2) (layer "B.Cu") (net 4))
 (segment (start 144.861845 51.107) (end 148.241845 54.487) (width 0.2) (layer "B.Cu") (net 3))
 (segment (start 148.241845 87.544) (end 144.300845 91.485) (width 0.2) (layer "B.Cu") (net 3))
 (segment (start 148.241845 54.487) (end 148.241845 87.544) (width 0.2) (layer "B.Cu") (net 3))
 (segment (start 132.190845 91.485) (end 128.120845 95.555) (width 0.2) (layer "B.Cu") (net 3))
 (segment (start 127.230845 49.63) (end 128.707845 51.107) (width 0.2) (layer "B.Cu") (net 3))
 (segment (start 144.300845 91.485) (end 132.190845 91.485) (width 0.2) (layer "B.Cu") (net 3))
 (segment (start 128.340845 95.775) (end 128.340845 100.935) (width 0.2) (layer "B.Cu") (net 3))
 (segment (start 128.120845 95.555) (end 128.340845 95.775) (width 0.2) (layer "B.Cu") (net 3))
 (segment (start 128.707845 51.107) (end 144.861845 51.107) (width 0.2) (layer "B.Cu") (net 3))
 (segment (start 138.260987 99.51525) (end 144.141845 105.396108) (width 0.2) (layer "F.Cu") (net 5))
 (segment (start 144.141845 106.473892) (end 132.229737 118.386) (width 0.2) (layer "F.Cu") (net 5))
 (segment (start 69.238745 39.47) (end 127.230845 39.47) (width 0.2) (layer "F.Cu") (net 5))
 (segment (start 66.579845 115.2411) (end 66.579845 42.1289) (width 0.2) (layer "F.Cu") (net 5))
 (segment (start 66.579845 42.1289) (end 69.238745 39.47) (width 0.2) (layer "F.Cu") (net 5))
 (segment (start 69.724745 118.386) (end 66.579845 115.2411) (width 0.2) (layer "F.Cu") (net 5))
 (segment (start 144.141845 105.396108) (end 144.141845 106.473892) (width 0.2) (layer "F.Cu") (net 5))
 (segment (start 120.138345 99.6) (end 118.922095 100.81625) (width 0.2) (layer "F.Cu") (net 5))
 (segment (start 142.840845 100.935) (end 141.505845 99.6) (width 0.2) (layer "F.Cu") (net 5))
 (segment (start 132.229737 118.386) (end 69.724745 118.386) (width 0.2) (layer "F.Cu") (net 5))
 (segment (start 120.223095 99.51525) (end 138.260987 99.51525) (width 0.2) (layer "F.Cu") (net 5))
 (segment (start 141.505845 99.6) (end 120.138345 99.6) (width 0.2) (layer "F.Cu") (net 5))
 (segment (start 118.922095 100.81625) (end 120.223095 99.51525) (width 0.2) (layer "F.Cu") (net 5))
 (segment (start 127.230845 39.47) (end 126.645845 38.885) (width 0.2) (layer "F.Cu") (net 5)))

